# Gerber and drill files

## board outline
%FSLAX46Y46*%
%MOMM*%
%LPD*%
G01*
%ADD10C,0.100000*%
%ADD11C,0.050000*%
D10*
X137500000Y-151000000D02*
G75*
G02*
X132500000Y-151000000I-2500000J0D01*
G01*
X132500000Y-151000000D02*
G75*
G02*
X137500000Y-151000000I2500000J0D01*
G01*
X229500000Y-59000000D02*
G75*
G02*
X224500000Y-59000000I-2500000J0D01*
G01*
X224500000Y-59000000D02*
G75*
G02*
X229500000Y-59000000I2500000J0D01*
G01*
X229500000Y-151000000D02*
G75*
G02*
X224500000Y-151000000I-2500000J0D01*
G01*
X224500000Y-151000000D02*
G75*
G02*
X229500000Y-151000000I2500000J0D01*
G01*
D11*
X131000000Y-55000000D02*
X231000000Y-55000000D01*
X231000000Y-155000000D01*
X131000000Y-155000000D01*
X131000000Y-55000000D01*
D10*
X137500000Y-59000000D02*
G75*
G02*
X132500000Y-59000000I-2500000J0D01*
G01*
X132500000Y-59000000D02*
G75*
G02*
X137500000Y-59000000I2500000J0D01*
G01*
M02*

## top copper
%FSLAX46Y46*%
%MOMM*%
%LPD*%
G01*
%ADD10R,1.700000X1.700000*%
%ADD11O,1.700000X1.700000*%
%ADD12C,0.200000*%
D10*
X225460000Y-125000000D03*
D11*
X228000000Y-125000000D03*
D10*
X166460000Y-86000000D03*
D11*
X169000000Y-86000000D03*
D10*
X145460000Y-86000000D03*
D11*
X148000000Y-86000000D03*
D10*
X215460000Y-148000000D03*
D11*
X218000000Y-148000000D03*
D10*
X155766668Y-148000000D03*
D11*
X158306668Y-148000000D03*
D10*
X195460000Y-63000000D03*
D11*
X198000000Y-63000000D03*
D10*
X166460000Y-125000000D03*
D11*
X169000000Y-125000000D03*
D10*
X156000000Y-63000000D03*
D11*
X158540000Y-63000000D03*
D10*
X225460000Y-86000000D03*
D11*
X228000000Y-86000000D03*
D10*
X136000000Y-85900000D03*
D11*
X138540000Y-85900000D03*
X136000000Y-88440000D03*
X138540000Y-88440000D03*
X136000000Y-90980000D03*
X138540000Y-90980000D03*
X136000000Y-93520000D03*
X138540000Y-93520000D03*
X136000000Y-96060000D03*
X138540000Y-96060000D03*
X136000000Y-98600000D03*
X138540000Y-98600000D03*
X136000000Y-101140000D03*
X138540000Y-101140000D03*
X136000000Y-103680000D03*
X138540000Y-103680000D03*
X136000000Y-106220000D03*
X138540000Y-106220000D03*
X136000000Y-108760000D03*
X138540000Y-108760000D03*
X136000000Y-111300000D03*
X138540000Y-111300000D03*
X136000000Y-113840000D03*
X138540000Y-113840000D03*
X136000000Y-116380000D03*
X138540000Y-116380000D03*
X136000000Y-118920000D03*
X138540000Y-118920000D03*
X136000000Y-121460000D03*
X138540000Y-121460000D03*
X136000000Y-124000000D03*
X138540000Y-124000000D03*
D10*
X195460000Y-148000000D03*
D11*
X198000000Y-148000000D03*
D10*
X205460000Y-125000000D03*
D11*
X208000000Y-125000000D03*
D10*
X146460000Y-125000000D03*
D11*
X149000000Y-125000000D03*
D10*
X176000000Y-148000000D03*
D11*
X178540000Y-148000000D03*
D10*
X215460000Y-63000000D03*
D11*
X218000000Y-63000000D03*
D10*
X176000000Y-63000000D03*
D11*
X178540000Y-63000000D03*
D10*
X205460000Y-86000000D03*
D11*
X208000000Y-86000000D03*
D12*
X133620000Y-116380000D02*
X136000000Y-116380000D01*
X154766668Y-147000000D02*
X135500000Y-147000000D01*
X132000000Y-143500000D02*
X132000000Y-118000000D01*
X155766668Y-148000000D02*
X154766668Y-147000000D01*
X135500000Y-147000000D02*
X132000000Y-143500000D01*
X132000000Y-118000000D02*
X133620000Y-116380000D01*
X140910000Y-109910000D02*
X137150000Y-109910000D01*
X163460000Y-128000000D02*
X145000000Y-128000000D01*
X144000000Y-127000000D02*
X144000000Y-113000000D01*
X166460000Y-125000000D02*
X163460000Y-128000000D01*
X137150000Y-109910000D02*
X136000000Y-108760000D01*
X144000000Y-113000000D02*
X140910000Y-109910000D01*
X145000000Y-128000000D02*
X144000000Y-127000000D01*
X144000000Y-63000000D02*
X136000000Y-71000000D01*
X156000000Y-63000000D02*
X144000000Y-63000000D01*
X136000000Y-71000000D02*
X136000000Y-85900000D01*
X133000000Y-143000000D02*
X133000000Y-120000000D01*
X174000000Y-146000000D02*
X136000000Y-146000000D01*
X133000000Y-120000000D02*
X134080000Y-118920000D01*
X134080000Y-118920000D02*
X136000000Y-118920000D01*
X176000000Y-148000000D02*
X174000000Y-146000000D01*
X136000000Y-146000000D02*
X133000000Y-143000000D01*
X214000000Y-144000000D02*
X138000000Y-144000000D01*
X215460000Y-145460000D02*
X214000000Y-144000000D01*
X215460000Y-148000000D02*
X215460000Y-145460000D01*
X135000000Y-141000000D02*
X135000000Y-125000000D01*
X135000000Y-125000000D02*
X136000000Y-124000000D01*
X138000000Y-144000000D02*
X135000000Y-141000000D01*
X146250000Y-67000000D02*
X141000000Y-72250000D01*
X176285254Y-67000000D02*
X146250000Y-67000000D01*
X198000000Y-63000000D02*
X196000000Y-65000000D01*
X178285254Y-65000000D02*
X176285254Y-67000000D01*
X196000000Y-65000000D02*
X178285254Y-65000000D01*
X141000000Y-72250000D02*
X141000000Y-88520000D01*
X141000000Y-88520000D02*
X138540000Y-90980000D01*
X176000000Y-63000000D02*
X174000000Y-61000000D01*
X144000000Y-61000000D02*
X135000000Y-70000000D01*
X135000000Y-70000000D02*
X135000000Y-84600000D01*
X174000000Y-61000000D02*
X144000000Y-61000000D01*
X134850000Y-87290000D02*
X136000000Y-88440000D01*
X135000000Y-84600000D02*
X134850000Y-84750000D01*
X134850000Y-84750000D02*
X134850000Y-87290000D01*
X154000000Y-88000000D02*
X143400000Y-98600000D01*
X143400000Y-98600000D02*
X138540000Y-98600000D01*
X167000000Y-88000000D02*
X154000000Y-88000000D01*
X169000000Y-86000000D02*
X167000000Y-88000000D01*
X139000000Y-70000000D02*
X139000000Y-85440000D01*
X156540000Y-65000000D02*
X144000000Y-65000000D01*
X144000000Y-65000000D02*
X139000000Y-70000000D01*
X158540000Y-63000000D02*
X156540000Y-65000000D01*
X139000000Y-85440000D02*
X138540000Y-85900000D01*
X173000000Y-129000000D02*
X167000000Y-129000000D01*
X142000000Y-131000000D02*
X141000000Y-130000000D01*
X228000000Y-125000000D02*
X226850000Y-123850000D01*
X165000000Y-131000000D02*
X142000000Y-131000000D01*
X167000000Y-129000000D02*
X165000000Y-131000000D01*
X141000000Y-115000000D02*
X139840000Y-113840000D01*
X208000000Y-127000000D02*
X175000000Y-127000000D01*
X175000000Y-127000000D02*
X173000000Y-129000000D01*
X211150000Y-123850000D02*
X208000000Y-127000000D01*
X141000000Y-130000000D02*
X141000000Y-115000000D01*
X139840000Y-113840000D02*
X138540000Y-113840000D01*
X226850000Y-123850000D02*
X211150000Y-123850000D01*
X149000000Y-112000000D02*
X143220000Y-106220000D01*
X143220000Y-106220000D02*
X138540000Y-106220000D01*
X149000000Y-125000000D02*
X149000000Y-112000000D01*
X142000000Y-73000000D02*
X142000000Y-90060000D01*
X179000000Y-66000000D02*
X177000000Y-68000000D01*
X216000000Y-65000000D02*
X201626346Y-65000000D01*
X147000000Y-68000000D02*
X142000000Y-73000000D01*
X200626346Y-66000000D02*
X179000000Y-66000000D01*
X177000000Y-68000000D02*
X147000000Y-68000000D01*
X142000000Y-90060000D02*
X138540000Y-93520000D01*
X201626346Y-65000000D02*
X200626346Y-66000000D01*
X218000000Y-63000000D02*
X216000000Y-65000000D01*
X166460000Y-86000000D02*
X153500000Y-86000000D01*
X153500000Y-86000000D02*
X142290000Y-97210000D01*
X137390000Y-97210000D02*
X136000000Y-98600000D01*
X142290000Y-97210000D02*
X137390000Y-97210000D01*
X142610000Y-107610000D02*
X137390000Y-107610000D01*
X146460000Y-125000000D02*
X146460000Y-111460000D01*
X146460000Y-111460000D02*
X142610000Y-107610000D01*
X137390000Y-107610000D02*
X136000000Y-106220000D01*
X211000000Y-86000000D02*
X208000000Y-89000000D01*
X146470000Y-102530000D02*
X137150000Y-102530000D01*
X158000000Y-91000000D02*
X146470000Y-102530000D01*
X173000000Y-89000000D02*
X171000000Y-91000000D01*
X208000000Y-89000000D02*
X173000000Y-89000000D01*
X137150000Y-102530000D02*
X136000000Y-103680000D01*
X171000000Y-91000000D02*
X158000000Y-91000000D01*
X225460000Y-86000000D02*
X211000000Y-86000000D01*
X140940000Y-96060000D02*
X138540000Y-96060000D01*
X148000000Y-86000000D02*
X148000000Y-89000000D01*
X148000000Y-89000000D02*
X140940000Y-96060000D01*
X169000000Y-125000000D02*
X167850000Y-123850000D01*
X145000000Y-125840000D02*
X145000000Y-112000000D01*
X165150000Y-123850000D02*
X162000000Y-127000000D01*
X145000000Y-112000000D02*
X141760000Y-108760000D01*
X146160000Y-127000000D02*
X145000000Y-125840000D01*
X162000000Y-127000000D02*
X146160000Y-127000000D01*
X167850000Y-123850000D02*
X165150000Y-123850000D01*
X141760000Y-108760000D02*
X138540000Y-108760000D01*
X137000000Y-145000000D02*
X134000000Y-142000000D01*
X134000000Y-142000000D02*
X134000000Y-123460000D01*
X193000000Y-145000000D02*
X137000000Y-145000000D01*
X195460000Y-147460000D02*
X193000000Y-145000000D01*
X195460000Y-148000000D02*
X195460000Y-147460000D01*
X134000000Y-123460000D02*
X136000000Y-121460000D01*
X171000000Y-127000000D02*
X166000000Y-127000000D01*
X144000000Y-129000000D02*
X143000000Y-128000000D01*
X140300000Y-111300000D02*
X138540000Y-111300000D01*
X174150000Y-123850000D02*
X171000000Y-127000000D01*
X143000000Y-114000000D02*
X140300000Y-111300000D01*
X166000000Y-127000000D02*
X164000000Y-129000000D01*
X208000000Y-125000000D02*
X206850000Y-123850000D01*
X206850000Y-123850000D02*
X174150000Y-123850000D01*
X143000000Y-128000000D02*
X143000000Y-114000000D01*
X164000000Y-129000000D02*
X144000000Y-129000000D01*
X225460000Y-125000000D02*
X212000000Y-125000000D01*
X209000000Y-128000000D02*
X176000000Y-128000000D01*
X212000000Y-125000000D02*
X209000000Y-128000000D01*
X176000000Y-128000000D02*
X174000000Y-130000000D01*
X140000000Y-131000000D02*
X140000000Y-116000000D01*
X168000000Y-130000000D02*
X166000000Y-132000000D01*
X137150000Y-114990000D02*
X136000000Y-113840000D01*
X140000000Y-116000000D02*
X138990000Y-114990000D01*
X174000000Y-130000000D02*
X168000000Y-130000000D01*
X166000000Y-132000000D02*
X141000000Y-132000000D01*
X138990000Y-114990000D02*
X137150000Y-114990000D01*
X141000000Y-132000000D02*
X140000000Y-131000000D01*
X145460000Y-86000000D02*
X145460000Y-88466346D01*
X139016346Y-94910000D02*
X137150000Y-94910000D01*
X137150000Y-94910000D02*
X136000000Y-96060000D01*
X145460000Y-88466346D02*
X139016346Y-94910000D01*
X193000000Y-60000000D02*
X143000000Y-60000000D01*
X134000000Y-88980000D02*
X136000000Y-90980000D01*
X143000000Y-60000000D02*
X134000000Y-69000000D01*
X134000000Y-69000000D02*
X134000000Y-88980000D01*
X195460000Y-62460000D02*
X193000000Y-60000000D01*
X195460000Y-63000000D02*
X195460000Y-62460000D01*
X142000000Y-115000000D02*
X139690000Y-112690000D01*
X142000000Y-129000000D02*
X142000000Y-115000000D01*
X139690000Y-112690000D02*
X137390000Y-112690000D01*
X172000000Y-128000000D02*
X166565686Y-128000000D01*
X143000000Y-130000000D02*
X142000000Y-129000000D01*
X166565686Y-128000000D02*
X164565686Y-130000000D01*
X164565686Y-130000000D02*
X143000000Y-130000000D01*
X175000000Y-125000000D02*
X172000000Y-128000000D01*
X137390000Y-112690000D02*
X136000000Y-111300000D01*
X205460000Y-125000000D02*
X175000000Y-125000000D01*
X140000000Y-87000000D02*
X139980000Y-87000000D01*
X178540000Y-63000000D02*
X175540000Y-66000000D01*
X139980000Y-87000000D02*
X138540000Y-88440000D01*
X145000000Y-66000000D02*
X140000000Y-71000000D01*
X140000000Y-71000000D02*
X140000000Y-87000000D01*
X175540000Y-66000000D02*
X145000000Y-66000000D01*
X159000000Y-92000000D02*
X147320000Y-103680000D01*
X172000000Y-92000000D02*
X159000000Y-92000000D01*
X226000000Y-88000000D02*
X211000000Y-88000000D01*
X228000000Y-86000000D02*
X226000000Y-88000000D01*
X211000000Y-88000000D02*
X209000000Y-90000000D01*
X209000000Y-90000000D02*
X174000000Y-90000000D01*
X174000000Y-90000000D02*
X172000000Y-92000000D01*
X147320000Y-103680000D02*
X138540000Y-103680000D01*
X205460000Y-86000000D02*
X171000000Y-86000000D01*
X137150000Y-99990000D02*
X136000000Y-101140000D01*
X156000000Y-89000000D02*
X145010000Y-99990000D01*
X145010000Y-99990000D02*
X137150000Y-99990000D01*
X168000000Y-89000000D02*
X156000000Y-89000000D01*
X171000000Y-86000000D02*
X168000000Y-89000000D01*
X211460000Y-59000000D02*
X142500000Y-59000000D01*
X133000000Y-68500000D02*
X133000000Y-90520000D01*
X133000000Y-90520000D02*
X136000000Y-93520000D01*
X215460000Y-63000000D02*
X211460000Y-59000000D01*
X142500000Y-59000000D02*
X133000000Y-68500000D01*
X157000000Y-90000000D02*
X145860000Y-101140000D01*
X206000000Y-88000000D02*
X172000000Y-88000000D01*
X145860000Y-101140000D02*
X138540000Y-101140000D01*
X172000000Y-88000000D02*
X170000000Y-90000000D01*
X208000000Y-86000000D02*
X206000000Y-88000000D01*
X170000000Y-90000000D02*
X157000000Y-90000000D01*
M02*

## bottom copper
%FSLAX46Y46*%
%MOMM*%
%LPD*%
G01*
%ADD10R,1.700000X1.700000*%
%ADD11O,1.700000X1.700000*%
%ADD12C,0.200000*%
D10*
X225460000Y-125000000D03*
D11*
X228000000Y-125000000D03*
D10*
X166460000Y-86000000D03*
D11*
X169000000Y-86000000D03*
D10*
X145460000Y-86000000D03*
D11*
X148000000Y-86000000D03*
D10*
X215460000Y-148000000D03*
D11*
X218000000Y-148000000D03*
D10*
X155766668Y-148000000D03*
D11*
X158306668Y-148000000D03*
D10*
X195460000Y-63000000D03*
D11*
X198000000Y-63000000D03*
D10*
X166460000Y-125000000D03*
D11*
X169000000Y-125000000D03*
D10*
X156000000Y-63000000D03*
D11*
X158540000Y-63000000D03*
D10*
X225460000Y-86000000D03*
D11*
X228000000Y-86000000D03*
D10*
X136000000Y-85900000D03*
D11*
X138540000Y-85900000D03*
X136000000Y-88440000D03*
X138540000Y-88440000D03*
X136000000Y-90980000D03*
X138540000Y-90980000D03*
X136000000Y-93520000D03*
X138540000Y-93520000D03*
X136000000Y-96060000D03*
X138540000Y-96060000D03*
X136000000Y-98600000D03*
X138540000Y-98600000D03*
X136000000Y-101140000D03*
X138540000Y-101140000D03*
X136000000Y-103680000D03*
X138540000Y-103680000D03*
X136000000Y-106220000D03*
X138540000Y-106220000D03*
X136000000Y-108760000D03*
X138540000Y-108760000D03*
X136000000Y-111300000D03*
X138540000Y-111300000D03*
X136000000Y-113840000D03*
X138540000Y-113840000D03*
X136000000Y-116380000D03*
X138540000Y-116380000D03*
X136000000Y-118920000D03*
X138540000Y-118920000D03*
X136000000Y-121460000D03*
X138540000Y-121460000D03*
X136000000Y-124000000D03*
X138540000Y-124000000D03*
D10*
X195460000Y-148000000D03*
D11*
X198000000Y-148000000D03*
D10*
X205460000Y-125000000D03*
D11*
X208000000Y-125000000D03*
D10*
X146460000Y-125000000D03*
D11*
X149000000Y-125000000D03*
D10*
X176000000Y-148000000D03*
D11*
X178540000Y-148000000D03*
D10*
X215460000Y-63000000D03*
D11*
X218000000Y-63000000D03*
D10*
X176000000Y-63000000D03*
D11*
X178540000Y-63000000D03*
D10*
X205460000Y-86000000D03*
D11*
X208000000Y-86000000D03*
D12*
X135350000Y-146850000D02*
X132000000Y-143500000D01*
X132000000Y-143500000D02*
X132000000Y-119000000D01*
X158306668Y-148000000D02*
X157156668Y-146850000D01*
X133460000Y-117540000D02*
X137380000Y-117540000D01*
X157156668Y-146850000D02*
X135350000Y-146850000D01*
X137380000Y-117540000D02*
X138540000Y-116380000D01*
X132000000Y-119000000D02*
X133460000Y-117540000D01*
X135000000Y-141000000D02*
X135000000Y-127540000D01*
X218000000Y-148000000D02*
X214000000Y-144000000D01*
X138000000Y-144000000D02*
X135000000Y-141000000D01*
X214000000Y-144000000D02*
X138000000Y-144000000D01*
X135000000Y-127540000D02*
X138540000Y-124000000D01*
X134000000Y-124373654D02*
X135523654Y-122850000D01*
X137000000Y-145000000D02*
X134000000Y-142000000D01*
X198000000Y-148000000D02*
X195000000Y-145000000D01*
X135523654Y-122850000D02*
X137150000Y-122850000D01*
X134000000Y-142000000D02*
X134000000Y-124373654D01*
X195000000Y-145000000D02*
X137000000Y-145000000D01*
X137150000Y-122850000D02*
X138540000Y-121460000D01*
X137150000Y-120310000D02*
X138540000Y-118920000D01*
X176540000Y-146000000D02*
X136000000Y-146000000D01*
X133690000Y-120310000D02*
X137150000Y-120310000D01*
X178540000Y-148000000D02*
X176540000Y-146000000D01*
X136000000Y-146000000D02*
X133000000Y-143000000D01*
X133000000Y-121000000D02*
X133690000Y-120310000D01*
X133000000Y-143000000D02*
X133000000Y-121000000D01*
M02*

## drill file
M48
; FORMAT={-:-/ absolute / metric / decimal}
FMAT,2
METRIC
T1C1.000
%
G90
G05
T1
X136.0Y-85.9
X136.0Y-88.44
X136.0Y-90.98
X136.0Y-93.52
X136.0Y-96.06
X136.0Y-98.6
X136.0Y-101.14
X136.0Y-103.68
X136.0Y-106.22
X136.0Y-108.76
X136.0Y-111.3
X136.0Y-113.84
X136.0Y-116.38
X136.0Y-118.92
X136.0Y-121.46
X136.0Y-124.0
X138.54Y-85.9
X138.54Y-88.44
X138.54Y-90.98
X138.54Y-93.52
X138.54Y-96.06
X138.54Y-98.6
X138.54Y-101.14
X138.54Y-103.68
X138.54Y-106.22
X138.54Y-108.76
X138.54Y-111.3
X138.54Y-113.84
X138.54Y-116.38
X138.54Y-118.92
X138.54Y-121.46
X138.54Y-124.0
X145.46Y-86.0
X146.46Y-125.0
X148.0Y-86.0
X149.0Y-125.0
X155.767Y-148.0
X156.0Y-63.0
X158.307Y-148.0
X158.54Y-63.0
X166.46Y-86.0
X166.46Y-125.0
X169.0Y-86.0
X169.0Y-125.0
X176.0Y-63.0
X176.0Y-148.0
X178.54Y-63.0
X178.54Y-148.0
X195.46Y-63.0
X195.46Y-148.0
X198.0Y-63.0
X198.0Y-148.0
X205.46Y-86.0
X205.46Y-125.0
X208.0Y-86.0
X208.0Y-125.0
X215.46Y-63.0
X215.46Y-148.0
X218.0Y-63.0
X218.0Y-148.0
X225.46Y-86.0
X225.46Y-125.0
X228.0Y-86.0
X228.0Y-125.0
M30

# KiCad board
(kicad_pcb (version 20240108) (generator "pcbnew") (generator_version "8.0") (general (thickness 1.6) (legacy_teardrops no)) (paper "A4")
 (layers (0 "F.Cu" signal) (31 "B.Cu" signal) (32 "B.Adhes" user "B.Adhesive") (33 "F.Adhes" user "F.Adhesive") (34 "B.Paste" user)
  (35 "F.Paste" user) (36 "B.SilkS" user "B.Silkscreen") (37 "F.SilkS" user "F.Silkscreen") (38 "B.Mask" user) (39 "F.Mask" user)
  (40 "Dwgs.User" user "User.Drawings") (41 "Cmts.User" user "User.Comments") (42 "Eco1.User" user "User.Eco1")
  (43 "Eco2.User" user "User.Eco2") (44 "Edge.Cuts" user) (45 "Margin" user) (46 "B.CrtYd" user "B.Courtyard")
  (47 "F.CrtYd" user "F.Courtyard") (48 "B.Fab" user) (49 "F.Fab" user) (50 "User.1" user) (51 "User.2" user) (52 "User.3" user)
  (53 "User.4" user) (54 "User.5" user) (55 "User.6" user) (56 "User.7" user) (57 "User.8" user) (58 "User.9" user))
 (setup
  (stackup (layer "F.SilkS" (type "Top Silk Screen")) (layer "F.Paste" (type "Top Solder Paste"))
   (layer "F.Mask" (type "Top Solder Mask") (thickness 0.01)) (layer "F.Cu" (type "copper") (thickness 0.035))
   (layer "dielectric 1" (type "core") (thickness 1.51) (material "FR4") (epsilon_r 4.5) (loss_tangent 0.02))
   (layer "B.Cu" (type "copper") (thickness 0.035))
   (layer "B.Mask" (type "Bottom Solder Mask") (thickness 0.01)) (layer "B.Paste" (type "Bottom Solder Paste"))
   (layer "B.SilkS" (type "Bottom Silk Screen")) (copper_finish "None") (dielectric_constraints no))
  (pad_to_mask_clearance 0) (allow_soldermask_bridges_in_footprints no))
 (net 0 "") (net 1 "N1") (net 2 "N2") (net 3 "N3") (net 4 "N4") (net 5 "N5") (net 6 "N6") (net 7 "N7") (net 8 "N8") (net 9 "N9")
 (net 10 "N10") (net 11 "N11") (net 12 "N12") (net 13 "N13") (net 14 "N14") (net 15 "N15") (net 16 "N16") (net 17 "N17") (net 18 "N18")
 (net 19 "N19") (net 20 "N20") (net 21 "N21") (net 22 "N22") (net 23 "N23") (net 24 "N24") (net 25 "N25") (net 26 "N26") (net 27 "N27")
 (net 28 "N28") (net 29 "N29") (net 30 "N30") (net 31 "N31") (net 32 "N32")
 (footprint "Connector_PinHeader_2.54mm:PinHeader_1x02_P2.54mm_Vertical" (layer "F.Cu") (at 225.46 125 90)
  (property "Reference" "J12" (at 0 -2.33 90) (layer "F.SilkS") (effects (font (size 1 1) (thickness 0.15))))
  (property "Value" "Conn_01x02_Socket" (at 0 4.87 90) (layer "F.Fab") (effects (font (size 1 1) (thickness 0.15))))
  (pad "1" thru_hole rect (at 0 0 90) (size 1.7 1.7) (drill 1) (layers "*.Cu" "*.Mask") (remove_unused_layers no) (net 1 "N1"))
  (pad "2" thru_hole oval (at 0 2.54 90) (size 1.7 1.7) (drill 1) (layers "*.Cu" "*.Mask") (remove_unused_layers no) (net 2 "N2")))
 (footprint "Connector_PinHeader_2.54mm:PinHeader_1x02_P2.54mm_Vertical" (layer "F.Cu") (at 166.46 86 90)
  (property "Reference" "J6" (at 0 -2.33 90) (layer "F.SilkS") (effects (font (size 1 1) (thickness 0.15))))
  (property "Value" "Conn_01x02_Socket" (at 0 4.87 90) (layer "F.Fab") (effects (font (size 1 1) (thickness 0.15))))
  (pad "1" thru_hole rect (at 0 0 90) (size 1.7 1.7) (drill 1) (layers "*.Cu" "*.Mask") (remove_unused_layers no) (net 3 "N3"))
  (pad "2" thru_hole oval (at 0 2.54 90) (size 1.7 1.7) (drill 1) (layers "*.Cu" "*.Mask") (remove_unused_layers no) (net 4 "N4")))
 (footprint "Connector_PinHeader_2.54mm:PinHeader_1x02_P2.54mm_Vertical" (layer "F.Cu") (at 145.46 86 90)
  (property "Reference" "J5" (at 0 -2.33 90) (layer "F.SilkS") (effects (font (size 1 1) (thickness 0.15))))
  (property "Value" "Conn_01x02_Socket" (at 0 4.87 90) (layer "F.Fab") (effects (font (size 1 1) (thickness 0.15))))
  (pad "1" thru_hole rect (at 0 0 90) (size 1.7 1.7) (drill 1) (layers "*.Cu" "*.Mask") (remove_unused_layers no) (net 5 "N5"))
  (pad "2" thru_hole oval (at 0 2.54 90) (size 1.7 1.7) (drill 1) (layers "*.Cu" "*.Mask") (remove_unused_layers no) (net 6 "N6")))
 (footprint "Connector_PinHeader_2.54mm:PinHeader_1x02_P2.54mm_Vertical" (layer "F.Cu") (at 215.46 148 90)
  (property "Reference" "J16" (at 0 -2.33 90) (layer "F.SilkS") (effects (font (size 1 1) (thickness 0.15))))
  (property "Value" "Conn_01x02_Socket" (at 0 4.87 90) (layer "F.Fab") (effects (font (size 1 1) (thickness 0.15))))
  (pad "1" thru_hole rect (at 0 0 90) (size 1.7 1.7) (drill 1) (layers "*.Cu" "*.Mask") (remove_unused_layers no) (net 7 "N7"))
  (pad "2" thru_hole oval (at 0 2.54 90) (size 1.7 1.7) (drill 1) (layers "*.Cu" "*.Mask") (remove_unused_layers no) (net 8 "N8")))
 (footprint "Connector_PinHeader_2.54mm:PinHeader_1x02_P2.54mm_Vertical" (layer "F.Cu") (at 155.766668 148 90)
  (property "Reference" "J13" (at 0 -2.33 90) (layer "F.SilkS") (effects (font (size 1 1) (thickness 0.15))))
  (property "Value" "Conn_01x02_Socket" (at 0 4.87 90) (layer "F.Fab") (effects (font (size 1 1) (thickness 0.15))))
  (pad "1" thru_hole rect (at 0 0 90) (size 1.7 1.7) (drill 1) (layers "*.Cu" "*.Mask") (remove_unused_layers no) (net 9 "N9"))
  (pad "2" thru_hole oval (at 0 2.54 90) (size 1.7 1.7) (drill 1) (layers "*.Cu" "*.Mask") (remove_unused_layers no) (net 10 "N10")))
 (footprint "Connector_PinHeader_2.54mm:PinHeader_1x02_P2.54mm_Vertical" (layer "F.Cu") (at 195.46 63 90)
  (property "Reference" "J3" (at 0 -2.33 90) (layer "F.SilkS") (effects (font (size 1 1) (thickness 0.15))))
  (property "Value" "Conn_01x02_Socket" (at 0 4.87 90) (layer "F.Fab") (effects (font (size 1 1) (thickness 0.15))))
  (pad "1" thru_hole rect (at 0 0 90) (size 1.7 1.7) (drill 1) (layers "*.Cu" "*.Mask") (remove_unused_layers no) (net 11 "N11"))
  (pad "2" thru_hole oval (at 0 2.54 90) (size 1.7 1.7) (drill 1) (layers "*.Cu" "*.Mask") (remove_unused_layers no) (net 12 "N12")))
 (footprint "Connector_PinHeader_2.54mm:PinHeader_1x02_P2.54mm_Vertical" (layer "F.Cu") (at 166.46 125 90)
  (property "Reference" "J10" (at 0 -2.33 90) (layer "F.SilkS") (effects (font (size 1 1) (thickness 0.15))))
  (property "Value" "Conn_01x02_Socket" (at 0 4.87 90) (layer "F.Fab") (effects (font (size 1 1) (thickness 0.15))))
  (pad "1" thru_hole rect (at 0 0 90) (size 1.7 1.7) (drill 1) (layers "*.Cu" "*.Mask") (remove_unused_layers no) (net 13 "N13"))
  (pad "2" thru_hole oval (at 0 2.54 90) (size 1.7 1.7) (drill 1) (layers "*.Cu" "*.Mask") (remove_unused_layers no) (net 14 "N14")))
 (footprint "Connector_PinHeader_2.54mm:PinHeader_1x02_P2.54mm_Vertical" (layer "F.Cu") (at 156 63 90)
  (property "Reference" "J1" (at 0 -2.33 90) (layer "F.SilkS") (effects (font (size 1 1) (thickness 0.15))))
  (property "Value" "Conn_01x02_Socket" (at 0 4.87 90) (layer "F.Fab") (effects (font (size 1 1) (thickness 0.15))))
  (pad "1" thru_hole rect (at 0 0 90) (size 1.7 1.7) (drill 1) (layers "*.Cu" "*.Mask") (remove_unused_layers no) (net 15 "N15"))
  (pad "2" thru_hole oval (at 0 2.54 90) (size 1.7 1.7) (drill 1) (layers "*.Cu" "*.Mask") (remove_unused_layers no) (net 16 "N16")))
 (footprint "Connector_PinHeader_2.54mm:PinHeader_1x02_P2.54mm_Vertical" (layer "F.Cu") (at 225.46 86 90)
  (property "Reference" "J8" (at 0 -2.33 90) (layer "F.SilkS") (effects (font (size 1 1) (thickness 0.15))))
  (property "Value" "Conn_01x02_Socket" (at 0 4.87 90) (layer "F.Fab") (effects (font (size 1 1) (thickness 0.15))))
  (pad "1" thru_hole rect (at 0 0 90) (size 1.7 1.7) (drill 1) (layers "*.Cu" "*.Mask") (remove_unused_layers no) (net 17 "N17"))
  (pad "2" thru_hole oval (at 0 2.54 90) (size 1.7 1.7) (drill 1) (layers "*.Cu" "*.Mask") (remove_unused_layers no) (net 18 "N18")))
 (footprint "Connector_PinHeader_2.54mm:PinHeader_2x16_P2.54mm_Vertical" (layer "F.Cu") (at 136 85.9)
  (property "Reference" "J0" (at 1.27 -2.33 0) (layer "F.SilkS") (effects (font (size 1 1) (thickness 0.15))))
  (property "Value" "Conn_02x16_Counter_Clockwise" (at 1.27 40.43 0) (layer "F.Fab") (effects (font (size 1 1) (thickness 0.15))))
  (pad "1" thru_hole rect (at 0 0) (size 1.7 1.7) (drill 1) (layers "*.Cu" "*.Mask") (remove_unused_layers no) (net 15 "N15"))
  (pad "2" thru_hole oval (at 2.54 0) (size 1.7 1.7) (drill 1) (layers "*.Cu" "*.Mask") (remove_unused_layers no) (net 16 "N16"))
  (pad "3" thru_hole oval (at 0 2.54) (size 1.7 1.7) (drill 1) (layers "*.Cu" "*.Mask") (remove_unused_layers no) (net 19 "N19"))
  (pad "4" thru_hole oval (at 2.54 2.54) (size 1.7 1.7) (drill 1) (layers "*.Cu" "*.Mask") (remove_unused_layers no) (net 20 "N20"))
  (pad "5" thru_hole oval (at 0 5.08) (size 1.7 1.7) (drill 1) (layers "*.Cu" "*.Mask") (remove_unused_layers no) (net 11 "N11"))
  (pad "6" thru_hole oval (at 2.54 5.08) (size 1.7 1.7) (drill 1) (layers "*.Cu" "*.Mask") (remove_unused_layers no) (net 12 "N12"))
  (pad "7" thru_hole oval (at 0 7.62) (size 1.7 1.7) (drill 1) (layers "*.Cu" "*.Mask") (remove_unused_layers no) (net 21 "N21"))
  (pad "8" thru_hole oval (at 2.54 7.62) (size 1.7 1.7) (drill 1) (layers "*.Cu" "*.Mask") (remove_unused_layers no) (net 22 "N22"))
  (pad "9" thru_hole oval (at 0 10.16) (size 1.7 1.7) (drill 1) (layers "*.Cu" "*.Mask") (remove_unused_layers no) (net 5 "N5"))
  (pad "10" thru_hole oval (at 2.54 10.16) (size 1.7 1.7) (drill 1) (layers "*.Cu" "*.Mask") (remove_unused_layers no) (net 6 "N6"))
  (pad "11" thru_hole oval (at 0 12.7) (size 1.7 1.7) (drill 1) (layers "*.Cu" "*.Mask") (remove_unused_layers no) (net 3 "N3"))
  (pad "12" thru_hole oval (at 2.54 12.7) (size 1.7 1.7) (drill 1) (layers "*.Cu" "*.Mask") (remove_unused_layers no) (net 4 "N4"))
  (pad "13" thru_hole oval (at 0 15.24) (size 1.7 1.7) (drill 1) (layers "*.Cu" "*.Mask") (remove_unused_layers no) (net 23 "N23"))
  (pad "14" thru_hole oval (at 2.54 15.24) (size 1.7 1.7) (drill 1) (layers "*.Cu" "*.Mask") (remove_unused_layers no) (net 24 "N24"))
  (pad "15" thru_hole oval (at 0 17.78) (size 1.7 1.7) (drill 1) (layers "*.Cu" "*.Mask") (remove_unused_layers no) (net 17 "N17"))
  (pad "16" thru_hole oval (at 2.54 17.78) (size 1.7 1.7) (drill 1) (layers "*.Cu" "*.Mask") (remove_unused_layers no) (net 18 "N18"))
  (pad "17" thru_hole oval (at 0 20.32) (size 1.7 1.7) (drill 1) (layers "*.Cu" "*.Mask") (remove_unused_layers no) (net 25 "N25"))
  (pad "18" thru_hole oval (at 2.54 20.32) (size 1.7 1.7) (drill 1) (layers "*.Cu" "*.Mask") (remove_unused_layers no) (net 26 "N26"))
  (pad "19" thru_hole oval (at 0 22.86) (size 1.7 1.7) (drill 1) (layers "*.Cu" "*.Mask") (remove_unused_layers no) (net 13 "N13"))
  (pad "20" thru_hole oval (at 2.54 22.86) (size 1.7 1.7) (drill 1) (layers "*.Cu" "*.Mask") (remove_unused_layers no) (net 14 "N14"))
  (pad "21" thru_hole oval (at 0 25.4) (size 1.7 1.7) (drill 1) (layers "*.Cu" "*.Mask") (remove_unused_layers no) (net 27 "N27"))
  (pad "22" thru_hole oval (at 2.54 25.4) (size 1.7 1.7) (drill 1) (layers "*.Cu" "*.Mask") (remove_unused_layers no) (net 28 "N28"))
  (pad "23" thru_hole oval (at 0 27.94) (size 1.7 1.7) (drill 1) (layers "*.Cu" "*.Mask") (remove_unused_layers no) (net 1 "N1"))
  (pad "24" thru_hole oval (at 2.54 27.94) (size 1.7 1.7) (drill 1) (layers "*.Cu" "*.Mask") (remove_unused_layers no) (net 2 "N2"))
  (pad "25" thru_hole oval (at 0 30.48) (size 1.7 1.7) (drill 1) (layers "*.Cu" "*.Mask") (remove_unused_layers no) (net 9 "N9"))
  (pad "26" thru_hole oval (at 2.54 30.48) (size 1.7 1.7) (drill 1) (layers "*.Cu" "*.Mask") (remove_unused_layers no) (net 10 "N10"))
  (pad "27" thru_hole oval (at 0 33.02) (size 1.7 1.7) (drill 1) (layers "*.Cu" "*.Mask") (remove_unused_layers no) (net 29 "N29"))
  (pad "28" thru_hole oval (at 2.54 33.02) (size 1.7 1.7) (drill 1) (layers "*.Cu" "*.Mask") (remove_unused_layers no) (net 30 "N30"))
  (pad "29" thru_hole oval (at 0 35.56) (size 1.7 1.7) (drill 1) (layers "*.Cu" "*.Mask") (remove_unused_layers no) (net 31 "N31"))
  (pad "30" thru_hole oval (at 2.54 35.56) (size 1.7 1.7) (drill 1) (layers "*.Cu" "*.Mask") (remove_unused_layers no) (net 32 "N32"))
  (pad "31" thru_hole oval (at 0 38.1) (size 1.7 1.7) (drill 1) (layers "*.Cu" "*.Mask") (remove_unused_layers no) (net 7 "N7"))
  (pad "32" thru_hole oval (at 2.54 38.1) (size 1.7 1.7) (drill 1) (layers "*.Cu" "*.Mask") (remove_unused_layers no) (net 8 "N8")))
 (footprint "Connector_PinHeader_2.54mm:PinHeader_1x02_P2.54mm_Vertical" (layer "F.Cu") (at 195.46 148 90)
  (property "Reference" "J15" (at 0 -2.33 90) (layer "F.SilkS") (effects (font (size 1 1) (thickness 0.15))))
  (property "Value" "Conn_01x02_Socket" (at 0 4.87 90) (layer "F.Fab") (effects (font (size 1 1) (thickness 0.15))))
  (pad "1" thru_hole rect (at 0 0 90) (size 1.7 1.7) (drill 1) (layers "*.Cu" "*.Mask") (remove_unused_layers no) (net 31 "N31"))
  (pad "2" thru_hole oval (at 0 2.54 90) (size 1.7 1.7) (drill 1) (layers "*.Cu" "*.Mask") (remove_unused_layers no) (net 32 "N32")))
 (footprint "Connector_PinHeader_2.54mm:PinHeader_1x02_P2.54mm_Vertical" (layer "F.Cu") (at 205.46 125 90)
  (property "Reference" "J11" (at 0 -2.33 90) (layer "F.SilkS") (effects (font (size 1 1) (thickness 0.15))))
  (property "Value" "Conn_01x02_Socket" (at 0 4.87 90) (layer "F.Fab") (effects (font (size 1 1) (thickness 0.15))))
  (pad "1" thru_hole rect (at 0 0 90) (size 1.7 1.7) (drill 1) (layers "*.Cu" "*.Mask") (remove_unused_layers no) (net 27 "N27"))
  (pad "2" thru_hole oval (at 0 2.54 90) (size 1.7 1.7) (drill 1) (layers "*.Cu" "*.Mask") (remove_unused_layers no) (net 28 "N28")))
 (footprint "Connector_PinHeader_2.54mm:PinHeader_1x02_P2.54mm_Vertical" (layer "F.Cu") (at 146.46 125 90)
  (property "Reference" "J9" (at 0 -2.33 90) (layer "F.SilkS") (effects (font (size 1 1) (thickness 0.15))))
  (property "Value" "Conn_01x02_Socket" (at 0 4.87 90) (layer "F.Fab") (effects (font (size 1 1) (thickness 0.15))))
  (pad "1" thru_hole rect (at 0 0 90) (size 1.7 1.7) (drill 1) (layers "*.Cu" "*.Mask") (remove_unused_layers no) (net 25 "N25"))
  (pad "2" thru_hole oval (at 0 2.54 90) (size 1.7 1.7) (drill 1) (layers "*.Cu" "*.Mask") (remove_unused_layers no) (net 26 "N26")))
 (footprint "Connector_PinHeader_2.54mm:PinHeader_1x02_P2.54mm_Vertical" (layer "F.Cu") (at 176 148 90)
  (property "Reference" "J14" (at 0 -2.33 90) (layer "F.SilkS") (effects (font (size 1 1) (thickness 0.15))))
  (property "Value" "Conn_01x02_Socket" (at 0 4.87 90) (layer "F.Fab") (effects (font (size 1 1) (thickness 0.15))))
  (pad "1" thru_hole rect (at 0 0 90) (size 1.7 1.7) (drill 1) (layers "*.Cu" "*.Mask") (remove_unused_layers no) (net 29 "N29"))
  (pad "2" thru_hole oval (at 0 2.54 90) (size 1.7 1.7) (drill 1) (layers "*.Cu" "*.Mask") (remove_unused_layers no) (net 30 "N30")))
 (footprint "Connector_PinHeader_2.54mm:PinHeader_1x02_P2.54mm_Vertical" (layer "F.Cu") (at 215.46 63 90)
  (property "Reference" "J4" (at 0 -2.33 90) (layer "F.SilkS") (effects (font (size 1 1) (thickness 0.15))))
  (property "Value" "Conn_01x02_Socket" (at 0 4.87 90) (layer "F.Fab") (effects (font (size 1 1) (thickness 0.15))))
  (pad "1" thru_hole rect (at 0 0 90) (size 1.7 1.7) (drill 1) (layers "*.Cu" "*.Mask") (remove_unused_layers no) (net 21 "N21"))
  (pad "2" thru_hole oval (at 0 2.54 90) (size 1.7 1.7) (drill 1) (layers "*.Cu" "*.Mask") (remove_unused_layers no) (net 22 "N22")))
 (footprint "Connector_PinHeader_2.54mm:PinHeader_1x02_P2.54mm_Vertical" (layer "F.Cu") (at 176 63 90)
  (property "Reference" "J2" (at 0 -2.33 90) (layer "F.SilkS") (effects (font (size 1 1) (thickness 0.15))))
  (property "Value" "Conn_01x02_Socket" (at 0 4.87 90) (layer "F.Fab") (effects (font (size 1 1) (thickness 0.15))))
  (pad "1" thru_hole rect (at 0 0 90) (size 1.7 1.7) (drill 1) (layers "*.Cu" "*.Mask") (remove_unused_layers no) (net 19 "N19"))
  (pad "2" thru_hole oval (at 0 2.54 90) (size 1.7 1.7) (drill 1) (layers "*.Cu" "*.Mask") (remove_unused_layers no) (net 20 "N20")))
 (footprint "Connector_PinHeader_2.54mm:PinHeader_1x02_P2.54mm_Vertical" (layer "F.Cu") (at 205.46 86 90)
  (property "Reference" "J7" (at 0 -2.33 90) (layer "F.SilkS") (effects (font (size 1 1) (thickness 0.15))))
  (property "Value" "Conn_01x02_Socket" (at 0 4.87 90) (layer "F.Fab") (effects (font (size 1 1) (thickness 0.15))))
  (pad "1" thru_hole rect (at 0 0 90) (size 1.7 1.7) (drill 1) (layers "*.Cu" "*.Mask") (remove_unused_layers no) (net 23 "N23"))
  (pad "2" thru_hole oval (at 0 2.54 90) (size 1.7 1.7) (drill 1) (layers "*.Cu" "*.Mask") (remove_unused_layers no) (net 24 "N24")))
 (gr_circle (center 135 151) (end 137.5 151) (stroke (width 0.1) (type default)) (fill none) (layer "Edge.Cuts"))
 (gr_circle (center 227 59) (end 229.5 59) (stroke (width 0.1) (type default)) (fill none) (layer "Edge.Cuts"))
 (gr_circle (center 227 151) (end 229.5 151) (stroke (width 0.1) (type default)) (fill none) (layer "Edge.Cuts"))
 (gr_rect (start 131 55) (end 231 155) (stroke (width 0.05) (type default)) (fill none) (layer "Edge.Cuts"))
 (gr_circle (center 135 59) (end 137.5 59) (stroke (width 0.1) (type default)) (fill none) (layer "Edge.Cuts"))
 (segment (start 133.62 116.38) (end 136 116.38) (width 0.2) (layer "F.Cu") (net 9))
 (segment (start 154.766668 147) (end 135.5 147) (width 0.2) (layer "F.Cu") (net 9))
 (segment (start 132 143.5) (end 132 118) (width 0.2) (layer "F.Cu") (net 9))
 (segment (start 155.766668 148) (end 154.766668 147) (width 0.2) (layer "F.Cu") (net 9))
 (segment (start 135.5 147) (end 132 143.5) (width 0.2) (layer "F.Cu") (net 9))
 (segment (start 132 118) (end 133.62 116.38) (width 0.2) (layer "F.Cu") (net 9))
 (segment (start 140.91 109.91) (end 137.15 109.91) (width 0.2) (layer "F.Cu") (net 13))
 (segment (start 163.46 128) (end 145 128) (width 0.2) (layer "F.Cu") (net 13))
 (segment (start 144 127) (end 144 113) (width 0.2) (layer "F.Cu") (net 13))
 (segment (start 166.46 125) (end 163.46 128) (width 0.2) (layer "F.Cu") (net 13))
 (segment (start 137.15 109.91) (end 136 108.76) (width 0.2) (layer "F.Cu") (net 13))
 (segment (start 144 113) (end 140.91 109.91) (width 0.2) (layer "F.Cu") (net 13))
 (segment (start 145 128) (end 144 127) (width 0.2) (layer "F.Cu") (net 13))
 (segment (start 144 63) (end 136 71) (width 0.2) (layer "F.Cu") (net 15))
 (segment (start 156 63) (end 144 63) (width 0.2) (layer "F.Cu") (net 15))
 (segment (start 136 71) (end 136 85.9) (width 0.2) (layer "F.Cu") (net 15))
 (segment (start 133 143) (end 133 120) (width 0.2) (layer "F.Cu") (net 29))
 (segment (start 174 146) (end 136 146) (width 0.2) (layer "F.Cu") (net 29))
 (segment (start 133 120) (end 134.08 118.92) (width 0.2) (layer "F.Cu") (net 29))
 (segment (start 134.08 118.92) (end 136 118.92) (width 0.2) (layer "F.Cu") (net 29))
 (segment (start 176 148) (end 174 146) (width 0.2) (layer "F.Cu") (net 29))
 (segment (start 136 146) (end 133 143) (width 0.2) (layer "F.Cu") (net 29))
 (segment (start 214 144) (end 138 144) (width 0.2) (layer "F.Cu") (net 7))
 (segment (start 215.46 145.46) (end 214 144) (width 0.2) (layer "F.Cu") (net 7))
 (segment (start 215.46 148) (end 215.46 145.46) (width 0.2) (layer "F.Cu") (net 7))
 (segment (start 135 141) (end 135 125) (width 0.2) (layer "F.Cu") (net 7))
 (segment (start 135 125) (end 136 124) (width 0.2) (layer "F.Cu") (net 7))
 (segment (start 138 144) (end 135 141) (width 0.2) (layer "F.Cu") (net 7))
 (segment (start 146.25 67) (end 141 72.25) (width 0.2) (layer "F.Cu") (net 12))
 (segment (start 176.285254 67) (end 146.25 67) (width 0.2) (layer "F.Cu") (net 12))
 (segment (start 198 63) (end 196 65) (width 0.2) (layer "F.Cu") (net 12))
 (segment (start 178.285254 65) (end 176.285254 67) (width 0.2) (layer "F.Cu") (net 12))
 (segment (start 196 65) (end 178.285254 65) (width 0.2) (layer "F.Cu") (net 12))
 (segment (start 141 72.25) (end 141 88.52) (width 0.2) (layer "F.Cu") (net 12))
 (segment (start 141 88.52) (end 138.54 90.98) (width 0.2) (layer "F.Cu") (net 12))
 (segment (start 176 63) (end 174 61) (width 0.2) (layer "F.Cu") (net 19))
 (segment (start 144 61) (end 135 70) (width 0.2) (layer "F.Cu") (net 19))
 (segment (start 135 70) (end 135 84.6) (width 0.2) (layer "F.Cu") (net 19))
 (segment (start 174 61) (end 144 61) (width 0.2) (layer "F.Cu") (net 19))
 (segment (start 134.85 87.29) (end 136 88.44) (width 0.2) (layer "F.Cu") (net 19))
 (segment (start 135 84.6) (end 134.85 84.75) (width 0.2) (layer "F.Cu") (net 19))
 (segment (start 134.85 84.75) (end 134.85 87.29) (width 0.2) (layer "F.Cu") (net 19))
 (segment (start 154 88) (end 143.4 98.6) (width 0.2) (layer "F.Cu") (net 4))
 (segment (start 143.4 98.6) (end 138.54 98.6) (width 0.2) (layer "F.Cu") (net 4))
 (segment (start 167 88) (end 154 88) (width 0.2) (layer "F.Cu") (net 4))
 (segment (start 169 86) (end 167 88) (width 0.2) (layer "F.Cu") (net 4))
 (segment (start 139 70) (end 139 85.44) (width 0.2) (layer "F.Cu") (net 16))
 (segment (start 156.54 65) (end 144 65) (width 0.2) (layer "F.Cu") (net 16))
 (segment (start 144 65) (end 139 70) (width 0.2) (layer "F.Cu") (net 16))
 (segment (start 158.54 63) (end 156.54 65) (width 0.2) (layer "F.Cu") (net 16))
 (segment (start 139 85.44) (end 138.54 85.9) (width 0.2) (layer "F.Cu") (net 16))
 (segment (start 173 129) (end 167 129) (width 0.2) (layer "F.Cu") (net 2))
 (segment (start 142 131) (end 141 130) (width 0.2) (layer "F.Cu") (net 2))
 (segment (start 228 125) (end 226.85 123.85) (width 0.2) (layer "F.Cu") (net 2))
 (segment (start 165 131) (end 142 131) (width 0.2) (layer "F.Cu") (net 2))
 (segment (start 167 129) (end 165 131) (width 0.2) (layer "F.Cu") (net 2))
 (segment (start 141 115) (end 139.84 113.84) (width 0.2) (layer "F.Cu") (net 2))
 (segment (start 208 127) (end 175 127) (width 0.2) (layer "F.Cu") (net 2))
 (segment (start 175 127) (end 173 129) (width 0.2) (layer "F.Cu") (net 2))
 (segment (start 211.15 123.85) (end 208 127) (width 0.2) (layer "F.Cu") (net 2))
 (segment (start 141 130) (end 141 115) (width 0.2) (layer "F.Cu") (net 2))
 (segment (start 139.84 113.84) (end 138.54 113.84) (width 0.2) (layer "F.Cu") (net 2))
 (segment (start 226.85 123.85) (end 211.15 123.85) (width 0.2) (layer "F.Cu") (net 2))
 (segment (start 149 112) (end 143.22 106.22) (width 0.2) (layer "F.Cu") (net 26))
 (segment (start 143.22 106.22) (end 138.54 106.22) (width 0.2) (layer "F.Cu") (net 26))
 (segment (start 149 125) (end 149 112) (width 0.2) (layer "F.Cu") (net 26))
 (segment (start 142 73) (end 142 90.06) (width 0.2) (layer "F.Cu") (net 22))
 (segment (start 179 66) (end 177 68) (width 0.2) (layer "F.Cu") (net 22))
 (segment (start 216 65) (end 201.626346 65) (width 0.2) (layer "F.Cu") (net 22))
 (segment (start 147 68) (end 142 73) (width 0.2) (layer "F.Cu") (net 22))
 (segment (start 200.626346 66) (end 179 66) (width 0.2) (layer "F.Cu") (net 22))
 (segment (start 177 68) (end 147 68) (width 0.2) (layer "F.Cu") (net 22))
 (segment (start 142 90.06) (end 138.54 93.52) (width 0.2) (layer "F.Cu") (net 22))
 (segment (start 201.626346 65) (end 200.626346 66) (width 0.2) (layer "F.Cu") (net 22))
 (segment (start 218 63) (end 216 65) (width 0.2) (layer "F.Cu") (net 22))
 (segment (start 166.46 86) (end 153.5 86) (width 0.2) (layer "F.Cu") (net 3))
 (segment (start 153.5 86) (end 142.29 97.21) (width 0.2) (layer "F.Cu") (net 3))
 (segment (start 137.39 97.21) (end 136 98.6) (width 0.2) (layer "F.Cu") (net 3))
 (segment (start 142.29 97.21) (end 137.39 97.21) (width 0.2) (layer "F.Cu") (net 3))
 (segment (start 135.35 146.85) (end 132 143.5) (width 0.2) (layer "B.Cu") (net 10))
 (segment (start 132 143.5) (end 132 119) (width 0.2) (layer "B.Cu") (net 10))
 (segment (start 158.306668 148) (end 157.156668 146.85) (width 0.2) (layer "B.Cu") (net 10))
 (segment (start 133.46 117.54) (end 137.38 117.54) (width 0.2) (layer "B.Cu") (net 10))
 (segment (start 157.156668 146.85) (end 135.35 146.85) (width 0.2) (layer "B.Cu") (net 10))
 (segment (start 137.38 117.54) (end 138.54 116.38) (width 0.2) (layer "B.Cu") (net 10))
 (segment (start 132 119) (end 133.46 117.54) (width 0.2) (layer "B.Cu") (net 10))
 (segment (start 142.61 107.61) (end 137.39 107.61) (width 0.2) (layer "F.Cu") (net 25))
 (segment (start 146.46 125) (end 146.46 111.46) (width 0.2) (layer "F.Cu") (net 25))
 (segment (start 146.46 111.46) (end 142.61 107.61) (width 0.2) (layer "F.Cu") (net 25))
 (segment (start 137.39 107.61) (end 136 106.22) (width 0.2) (layer "F.Cu") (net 25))
 (segment (start 211 86) (end 208 89) (width 0.2) (layer "F.Cu") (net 17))
 (segment (start 146.47 102.53) (end 137.15 102.53) (width 0.2) (layer "F.Cu") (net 17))
 (segment (start 158 91) (end 146.47 102.53) (width 0.2) (layer "F.Cu") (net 17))
 (segment (start 173 89) (end 171 91) (width 0.2) (layer "F.Cu") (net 17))
 (segment (start 208 89) (end 173 89) (width 0.2) (layer "F.Cu") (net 17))
 (segment (start 137.15 102.53) (end 136 103.68) (width 0.2) (layer "F.Cu") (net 17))
 (segment (start 171 91) (end 158 91) (width 0.2) (layer "F.Cu") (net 17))
 (segment (start 225.46 86) (end 211 86) (width 0.2) (layer "F.Cu") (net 17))
 (segment (start 140.94 96.06) (end 138.54 96.06) (width 0.2) (layer "F.Cu") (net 6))
 (segment (start 148 86) (end 148 89) (width 0.2) (layer "F.Cu") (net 6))
 (segment (start 148 89) (end 140.94 96.06) (width 0.2) (layer "F.Cu") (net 6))
 (segment (start 135 141) (end 135 127.54) (width 0.2) (layer "B.Cu") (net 8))
 (segment (start 218 148) (end 214 144) (width 0.2) (layer "B.Cu") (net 8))
 (segment (start 138 144) (end 135 141) (width 0.2) (layer "B.Cu") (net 8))
 (segment (start 214 144) (end 138 144) (width 0.2) (layer "B.Cu") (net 8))
 (segment (start 135 127.54) (end 138.54 124) (width 0.2) (layer "B.Cu") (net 8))
 (segment (start 134 124.373654) (end 135.523654 122.85) (width 0.2) (layer "B.Cu") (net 32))
 (segment (start 137 145) (end 134 142) (width 0.2) (layer "B.Cu") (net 32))
 (segment (start 198 148) (end 195 145) (width 0.2) (layer "B.Cu") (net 32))
 (segment (start 135.523654 122.85) (end 137.15 122.85) (width 0.2) (layer "B.Cu") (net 32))
 (segment (start 134 142) (end 134 124.373654) (width 0.2) (layer "B.Cu") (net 32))
 (segment (start 195 145) (end 137 145) (width 0.2) (layer "B.Cu") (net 32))
 (segment (start 137.15 122.85) (end 138.54 121.46) (width 0.2) (layer "B.Cu") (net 32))
 (segment (start 169 125) (end 167.85 123.85) (width 0.2) (layer "F.Cu") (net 14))
 (segment (start 145 125.84) (end 145 112) (width 0.2) (layer "F.Cu") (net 14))
 (segment (start 165.15 123.85) (end 162 127) (width 0.2) (layer "F.Cu") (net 14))
 (segment (start 145 112) (end 141.76 108.76) (width 0.2) (layer "F.Cu") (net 14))
 (segment (start 146.16 127) (end 145 125.84) (width 0.2) (layer "F.Cu") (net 14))
 (segment (start 162 127) (end 146.16 127) (width 0.2) (layer "F.Cu") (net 14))
 (segment (start 167.85 123.85) (end 165.15 123.85) (width 0.2) (layer "F.Cu") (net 14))
 (segment (start 141.76 108.76) (end 138.54 108.76) (width 0.2) (layer "F.Cu") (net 14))
 (segment (start 137 145) (end 134 142) (width 0.2) (layer "F.Cu") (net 31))
 (segment (start 134 142) (end 134 123.46) (width 0.2) (layer "F.Cu") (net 31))
 (segment (start 193 145) (end 137 145) (width 0.2) (layer "F.Cu") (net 31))
 (segment (start 195.46 147.46) (end 193 145) (width 0.2) (layer "F.Cu") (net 31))
 (segment (start 195.46 148) (end 195.46 147.46) (width 0.2) (layer "F.Cu") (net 31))
 (segment (start 134 123.46) (end 136 121.46) (width 0.2) (layer "F.Cu") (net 31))
 (segment (start 171 127) (end 166 127) (width 0.2) (layer "F.Cu") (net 28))
 (segment (start 144 129) (end 143 128) (width 0.2) (layer "F.Cu") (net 28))
 (segment (start 140.3 111.3) (end 138.54 111.3) (width 0.2) (layer "F.Cu") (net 28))
 (segment (start 174.15 123.85) (end 171 127) (width 0.2) (layer "F.Cu") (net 28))
 (segment (start 143 114) (end 140.3 111.3) (width 0.2) (layer "F.Cu") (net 28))
 (segment (start 166 127) (end 164 129) (width 0.2) (layer "F.Cu") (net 28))
 (segment (start 208 125) (end 206.85 123.85) (width 0.2) (layer "F.Cu") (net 28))
 (segment (start 206.85 123.85) (end 174.15 123.85) (width 0.2) (layer "F.Cu") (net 28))
 (segment (start 143 128) (end 143 114) (width 0.2) (layer "F.Cu") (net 28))
 (segment (start 164 129) (end 144 129) (width 0.2) (layer "F.Cu") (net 28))
 (segment (start 225.46 125) (end 212 125) (width 0.2) (layer "F.Cu") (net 1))
 (segment (start 209 128) (end 176 128) (width 0.2) (layer "F.Cu") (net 1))
 (segment (start 212 125) (end 209 128) (width 0.2) (layer "F.Cu") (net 1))
 (segment (start 176 128) (end 174 130) (width 0.2) (layer "F.Cu") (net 1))
 (segment (start 140 131) (end 140 116) (width 0.2) (layer "F.Cu") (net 1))
 (segment (start 168 130) (end 166 132) (width 0.2) (layer "F.Cu") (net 1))
 (segment (start 137.15 114.99) (end 136 113.84) (width 0.2) (layer "F.Cu") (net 1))
 (segment (start 140 116) (end 138.99 114.99) (width 0.2) (layer "F.Cu") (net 1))
 (segment (start 174 130) (end 168 130) (width 0.2) (layer "F.Cu") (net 1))
 (segment (start 166 132) (end 141 132) (width 0.2) (layer "F.Cu") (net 1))
 (segment (start 138.99 114.99) (end 137.15 114.99) (width 0.2) (layer "F.Cu") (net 1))
 (segment (start 141 132) (end 140 131) (width 0.2) (layer "F.Cu") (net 1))
 (segment (start 137.15 120.31) (end 138.54 118.92) (width 0.2) (layer "B.Cu") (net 30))
 (segment (start 176.54 146) (end 136 146) (width 0.2) (layer "B.Cu") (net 30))
 (segment (start 133.69 120.31) (end 137.15 120.31) (width 0.2) (layer "B.Cu") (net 30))
 (segment (start 178.54 148) (end 176.54 146) (width 0.2) (layer "B.Cu") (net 30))
 (segment (start 136 146) (end 133 143) (width 0.2) (layer "B.Cu") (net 30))
 (segment (start 133 121) (end 133.69 120.31) (width 0.2) (layer "B.Cu") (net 30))
 (segment (start 133 143) (end 133 121) (width 0.2) (layer "B.Cu") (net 30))
 (segment (start 145.46 86) (end 145.46 88.466346) (width 0.2) (layer "F.Cu") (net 5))
 (segment (start 139.016346 94.91) (end 137.15 94.91) (width 0.2) (layer "F.Cu") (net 5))
 (segment (start 137.15 94.91) (end 136 96.06) (width 0.2) (layer "F.Cu") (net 5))
 (segment (start 145.46 88.466346) (end 139.016346 94.91) (width 0.2) (layer "F.Cu") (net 5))
 (segment (start 193 60) (end 143 60) (width 0.2) (layer "F.Cu") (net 11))
 (segment (start 134 88.98) (end 136 90.98) (width 0.2) (layer "F.Cu") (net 11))
 (segment (start 143 60) (end 134 69) (width 0.2) (layer "F.Cu") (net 11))
 (segment (start 134 69) (end 134 88.98) (width 0.2) (layer "F.Cu") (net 11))
 (segment (start 195.46 62.46) (end 193 60) (width 0.2) (layer "F.Cu") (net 11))
 (segment (start 195.46 63) (end 195.46 62.46) (width 0.2) (layer "F.Cu") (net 11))
 (segment (start 142 115) (end 139.69 112.69) (width 0.2) (layer "F.Cu") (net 27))
 (segment (start 142 129) (end 142 115) (width 0.2) (layer "F.Cu") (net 27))
 (segment (start 139.69 112.69) (end 137.39 112.69) (width 0.2) (layer "F.Cu") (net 27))
 (segment (start 172 128) (end 166.565686 128) (width 0.2) (layer "F.Cu") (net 27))
 (segment (start 143 130) (end 142 129) (width 0.2) (layer "F.Cu") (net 27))
 (segment (start 166.565686 128) (end 164.565686 130) (width 0.2) (layer "F.Cu") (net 27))
 (segment (start 164.565686 130) (end 143 130) (width 0.2) (layer "F.Cu") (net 27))
 (segment (start 175 125) (end 172 128) (width 0.2) (layer "F.Cu") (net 27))
 (segment (start 137.39 112.69) (end 136 111.3) (width 0.2) (layer "F.Cu") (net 27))
 (segment (start 205.46 125) (end 175 125) (width 0.2) (layer "F.Cu") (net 27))
 (segment (start 140 87) (end 139.98 87) (width 0.2) (layer "F.Cu") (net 20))
 (segment (start 178.54 63) (end 175.54 66) (width 0.2) (layer "F.Cu") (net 20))
 (segment (start 139.98 87) (end 138.54 88.44) (width 0.2) (layer "F.Cu") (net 20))
 (segment (start 145 66) (end 140 71) (width 0.2) (layer "F.Cu") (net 20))
 (segment (start 140 71) (end 140 87) (width 0.2) (layer "F.Cu") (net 20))
 (segment (start 175.54 66) (end 145 66) (width 0.2) (layer "F.Cu") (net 20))
 (segment (start 159 92) (end 147.32 103.68) (width 0.2) (layer "F.Cu") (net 18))
 (segment (start 172 92) (end 159 92) (width 0.2) (layer "F.Cu") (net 18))
 (segment (start 226 88) (end 211 88) (width 0.2) (layer "F.Cu") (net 18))
 (segment (start 228 86) (end 226 88) (width 0.2) (layer "F.Cu") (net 18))
 (segment (start 211 88) (end 209 90) (width 0.2) (layer "F.Cu") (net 18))
 (segment (start 209 90) (end 174 90) (width 0.2) (layer "F.Cu") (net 18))
 (segment (start 174 90) (end 172 92) (width 0.2) (layer "F.Cu") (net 18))
 (segment (start 147.32 103.68) (end 138.54 103.68) (width 0.2) (layer "F.Cu") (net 18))
 (segment (start 205.46 86) (end 171 86) (width 0.2) (layer "F.Cu") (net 23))
 (segment (start 137.15 99.99) (end 136 101.14) (width 0.2) (layer "F.Cu") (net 23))
 (segment (start 156 89) (end 145.01 99.99) (width 0.2) (layer "F.Cu") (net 23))
 (segment (start 145.01 99.99) (end 137.15 99.99) (width 0.2) (layer "F.Cu") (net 23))
 (segment (start 168 89) (end 156 89) (width 0.2) (layer "F.Cu") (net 23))
 (segment (start 171 86) (end 168 89) (width 0.2) (layer "F.Cu") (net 23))
 (segment (start 211.46 59) (end 142.5 59) (width 0.2) (layer "F.Cu") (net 21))
 (segment (start 133 68.5) (end 133 90.52) (width 0.2) (layer "F.Cu") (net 21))
 (segment (start 133 90.52) (end 136 93.52) (width 0.2) (layer "F.Cu") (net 21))
 (segment (start 215.46 63) (end 211.46 59) (width 0.2) (layer "F.Cu") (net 21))
 (segment (start 142.5 59) (end 133 68.5) (width 0.2) (layer "F.Cu") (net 21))
 (segment (start 157 90) (end 145.86 101.14) (width 0.2) (layer "F.Cu") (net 24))
 (segment (start 206 88) (end 172 88) (width 0.2) (layer "F.Cu") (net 24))
 (segment (start 145.86 101.14) (end 138.54 101.14) (width 0.2) (layer "F.Cu") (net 24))
 (segment (start 172 88) (end 170 90) (width 0.2) (layer "F.Cu") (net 24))
 (segment (start 208 86) (end 206 88) (width 0.2) (layer "F.Cu") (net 24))
 (segment (start 170 90) (end 157 90) (width 0.2) (layer "F.Cu") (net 24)))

